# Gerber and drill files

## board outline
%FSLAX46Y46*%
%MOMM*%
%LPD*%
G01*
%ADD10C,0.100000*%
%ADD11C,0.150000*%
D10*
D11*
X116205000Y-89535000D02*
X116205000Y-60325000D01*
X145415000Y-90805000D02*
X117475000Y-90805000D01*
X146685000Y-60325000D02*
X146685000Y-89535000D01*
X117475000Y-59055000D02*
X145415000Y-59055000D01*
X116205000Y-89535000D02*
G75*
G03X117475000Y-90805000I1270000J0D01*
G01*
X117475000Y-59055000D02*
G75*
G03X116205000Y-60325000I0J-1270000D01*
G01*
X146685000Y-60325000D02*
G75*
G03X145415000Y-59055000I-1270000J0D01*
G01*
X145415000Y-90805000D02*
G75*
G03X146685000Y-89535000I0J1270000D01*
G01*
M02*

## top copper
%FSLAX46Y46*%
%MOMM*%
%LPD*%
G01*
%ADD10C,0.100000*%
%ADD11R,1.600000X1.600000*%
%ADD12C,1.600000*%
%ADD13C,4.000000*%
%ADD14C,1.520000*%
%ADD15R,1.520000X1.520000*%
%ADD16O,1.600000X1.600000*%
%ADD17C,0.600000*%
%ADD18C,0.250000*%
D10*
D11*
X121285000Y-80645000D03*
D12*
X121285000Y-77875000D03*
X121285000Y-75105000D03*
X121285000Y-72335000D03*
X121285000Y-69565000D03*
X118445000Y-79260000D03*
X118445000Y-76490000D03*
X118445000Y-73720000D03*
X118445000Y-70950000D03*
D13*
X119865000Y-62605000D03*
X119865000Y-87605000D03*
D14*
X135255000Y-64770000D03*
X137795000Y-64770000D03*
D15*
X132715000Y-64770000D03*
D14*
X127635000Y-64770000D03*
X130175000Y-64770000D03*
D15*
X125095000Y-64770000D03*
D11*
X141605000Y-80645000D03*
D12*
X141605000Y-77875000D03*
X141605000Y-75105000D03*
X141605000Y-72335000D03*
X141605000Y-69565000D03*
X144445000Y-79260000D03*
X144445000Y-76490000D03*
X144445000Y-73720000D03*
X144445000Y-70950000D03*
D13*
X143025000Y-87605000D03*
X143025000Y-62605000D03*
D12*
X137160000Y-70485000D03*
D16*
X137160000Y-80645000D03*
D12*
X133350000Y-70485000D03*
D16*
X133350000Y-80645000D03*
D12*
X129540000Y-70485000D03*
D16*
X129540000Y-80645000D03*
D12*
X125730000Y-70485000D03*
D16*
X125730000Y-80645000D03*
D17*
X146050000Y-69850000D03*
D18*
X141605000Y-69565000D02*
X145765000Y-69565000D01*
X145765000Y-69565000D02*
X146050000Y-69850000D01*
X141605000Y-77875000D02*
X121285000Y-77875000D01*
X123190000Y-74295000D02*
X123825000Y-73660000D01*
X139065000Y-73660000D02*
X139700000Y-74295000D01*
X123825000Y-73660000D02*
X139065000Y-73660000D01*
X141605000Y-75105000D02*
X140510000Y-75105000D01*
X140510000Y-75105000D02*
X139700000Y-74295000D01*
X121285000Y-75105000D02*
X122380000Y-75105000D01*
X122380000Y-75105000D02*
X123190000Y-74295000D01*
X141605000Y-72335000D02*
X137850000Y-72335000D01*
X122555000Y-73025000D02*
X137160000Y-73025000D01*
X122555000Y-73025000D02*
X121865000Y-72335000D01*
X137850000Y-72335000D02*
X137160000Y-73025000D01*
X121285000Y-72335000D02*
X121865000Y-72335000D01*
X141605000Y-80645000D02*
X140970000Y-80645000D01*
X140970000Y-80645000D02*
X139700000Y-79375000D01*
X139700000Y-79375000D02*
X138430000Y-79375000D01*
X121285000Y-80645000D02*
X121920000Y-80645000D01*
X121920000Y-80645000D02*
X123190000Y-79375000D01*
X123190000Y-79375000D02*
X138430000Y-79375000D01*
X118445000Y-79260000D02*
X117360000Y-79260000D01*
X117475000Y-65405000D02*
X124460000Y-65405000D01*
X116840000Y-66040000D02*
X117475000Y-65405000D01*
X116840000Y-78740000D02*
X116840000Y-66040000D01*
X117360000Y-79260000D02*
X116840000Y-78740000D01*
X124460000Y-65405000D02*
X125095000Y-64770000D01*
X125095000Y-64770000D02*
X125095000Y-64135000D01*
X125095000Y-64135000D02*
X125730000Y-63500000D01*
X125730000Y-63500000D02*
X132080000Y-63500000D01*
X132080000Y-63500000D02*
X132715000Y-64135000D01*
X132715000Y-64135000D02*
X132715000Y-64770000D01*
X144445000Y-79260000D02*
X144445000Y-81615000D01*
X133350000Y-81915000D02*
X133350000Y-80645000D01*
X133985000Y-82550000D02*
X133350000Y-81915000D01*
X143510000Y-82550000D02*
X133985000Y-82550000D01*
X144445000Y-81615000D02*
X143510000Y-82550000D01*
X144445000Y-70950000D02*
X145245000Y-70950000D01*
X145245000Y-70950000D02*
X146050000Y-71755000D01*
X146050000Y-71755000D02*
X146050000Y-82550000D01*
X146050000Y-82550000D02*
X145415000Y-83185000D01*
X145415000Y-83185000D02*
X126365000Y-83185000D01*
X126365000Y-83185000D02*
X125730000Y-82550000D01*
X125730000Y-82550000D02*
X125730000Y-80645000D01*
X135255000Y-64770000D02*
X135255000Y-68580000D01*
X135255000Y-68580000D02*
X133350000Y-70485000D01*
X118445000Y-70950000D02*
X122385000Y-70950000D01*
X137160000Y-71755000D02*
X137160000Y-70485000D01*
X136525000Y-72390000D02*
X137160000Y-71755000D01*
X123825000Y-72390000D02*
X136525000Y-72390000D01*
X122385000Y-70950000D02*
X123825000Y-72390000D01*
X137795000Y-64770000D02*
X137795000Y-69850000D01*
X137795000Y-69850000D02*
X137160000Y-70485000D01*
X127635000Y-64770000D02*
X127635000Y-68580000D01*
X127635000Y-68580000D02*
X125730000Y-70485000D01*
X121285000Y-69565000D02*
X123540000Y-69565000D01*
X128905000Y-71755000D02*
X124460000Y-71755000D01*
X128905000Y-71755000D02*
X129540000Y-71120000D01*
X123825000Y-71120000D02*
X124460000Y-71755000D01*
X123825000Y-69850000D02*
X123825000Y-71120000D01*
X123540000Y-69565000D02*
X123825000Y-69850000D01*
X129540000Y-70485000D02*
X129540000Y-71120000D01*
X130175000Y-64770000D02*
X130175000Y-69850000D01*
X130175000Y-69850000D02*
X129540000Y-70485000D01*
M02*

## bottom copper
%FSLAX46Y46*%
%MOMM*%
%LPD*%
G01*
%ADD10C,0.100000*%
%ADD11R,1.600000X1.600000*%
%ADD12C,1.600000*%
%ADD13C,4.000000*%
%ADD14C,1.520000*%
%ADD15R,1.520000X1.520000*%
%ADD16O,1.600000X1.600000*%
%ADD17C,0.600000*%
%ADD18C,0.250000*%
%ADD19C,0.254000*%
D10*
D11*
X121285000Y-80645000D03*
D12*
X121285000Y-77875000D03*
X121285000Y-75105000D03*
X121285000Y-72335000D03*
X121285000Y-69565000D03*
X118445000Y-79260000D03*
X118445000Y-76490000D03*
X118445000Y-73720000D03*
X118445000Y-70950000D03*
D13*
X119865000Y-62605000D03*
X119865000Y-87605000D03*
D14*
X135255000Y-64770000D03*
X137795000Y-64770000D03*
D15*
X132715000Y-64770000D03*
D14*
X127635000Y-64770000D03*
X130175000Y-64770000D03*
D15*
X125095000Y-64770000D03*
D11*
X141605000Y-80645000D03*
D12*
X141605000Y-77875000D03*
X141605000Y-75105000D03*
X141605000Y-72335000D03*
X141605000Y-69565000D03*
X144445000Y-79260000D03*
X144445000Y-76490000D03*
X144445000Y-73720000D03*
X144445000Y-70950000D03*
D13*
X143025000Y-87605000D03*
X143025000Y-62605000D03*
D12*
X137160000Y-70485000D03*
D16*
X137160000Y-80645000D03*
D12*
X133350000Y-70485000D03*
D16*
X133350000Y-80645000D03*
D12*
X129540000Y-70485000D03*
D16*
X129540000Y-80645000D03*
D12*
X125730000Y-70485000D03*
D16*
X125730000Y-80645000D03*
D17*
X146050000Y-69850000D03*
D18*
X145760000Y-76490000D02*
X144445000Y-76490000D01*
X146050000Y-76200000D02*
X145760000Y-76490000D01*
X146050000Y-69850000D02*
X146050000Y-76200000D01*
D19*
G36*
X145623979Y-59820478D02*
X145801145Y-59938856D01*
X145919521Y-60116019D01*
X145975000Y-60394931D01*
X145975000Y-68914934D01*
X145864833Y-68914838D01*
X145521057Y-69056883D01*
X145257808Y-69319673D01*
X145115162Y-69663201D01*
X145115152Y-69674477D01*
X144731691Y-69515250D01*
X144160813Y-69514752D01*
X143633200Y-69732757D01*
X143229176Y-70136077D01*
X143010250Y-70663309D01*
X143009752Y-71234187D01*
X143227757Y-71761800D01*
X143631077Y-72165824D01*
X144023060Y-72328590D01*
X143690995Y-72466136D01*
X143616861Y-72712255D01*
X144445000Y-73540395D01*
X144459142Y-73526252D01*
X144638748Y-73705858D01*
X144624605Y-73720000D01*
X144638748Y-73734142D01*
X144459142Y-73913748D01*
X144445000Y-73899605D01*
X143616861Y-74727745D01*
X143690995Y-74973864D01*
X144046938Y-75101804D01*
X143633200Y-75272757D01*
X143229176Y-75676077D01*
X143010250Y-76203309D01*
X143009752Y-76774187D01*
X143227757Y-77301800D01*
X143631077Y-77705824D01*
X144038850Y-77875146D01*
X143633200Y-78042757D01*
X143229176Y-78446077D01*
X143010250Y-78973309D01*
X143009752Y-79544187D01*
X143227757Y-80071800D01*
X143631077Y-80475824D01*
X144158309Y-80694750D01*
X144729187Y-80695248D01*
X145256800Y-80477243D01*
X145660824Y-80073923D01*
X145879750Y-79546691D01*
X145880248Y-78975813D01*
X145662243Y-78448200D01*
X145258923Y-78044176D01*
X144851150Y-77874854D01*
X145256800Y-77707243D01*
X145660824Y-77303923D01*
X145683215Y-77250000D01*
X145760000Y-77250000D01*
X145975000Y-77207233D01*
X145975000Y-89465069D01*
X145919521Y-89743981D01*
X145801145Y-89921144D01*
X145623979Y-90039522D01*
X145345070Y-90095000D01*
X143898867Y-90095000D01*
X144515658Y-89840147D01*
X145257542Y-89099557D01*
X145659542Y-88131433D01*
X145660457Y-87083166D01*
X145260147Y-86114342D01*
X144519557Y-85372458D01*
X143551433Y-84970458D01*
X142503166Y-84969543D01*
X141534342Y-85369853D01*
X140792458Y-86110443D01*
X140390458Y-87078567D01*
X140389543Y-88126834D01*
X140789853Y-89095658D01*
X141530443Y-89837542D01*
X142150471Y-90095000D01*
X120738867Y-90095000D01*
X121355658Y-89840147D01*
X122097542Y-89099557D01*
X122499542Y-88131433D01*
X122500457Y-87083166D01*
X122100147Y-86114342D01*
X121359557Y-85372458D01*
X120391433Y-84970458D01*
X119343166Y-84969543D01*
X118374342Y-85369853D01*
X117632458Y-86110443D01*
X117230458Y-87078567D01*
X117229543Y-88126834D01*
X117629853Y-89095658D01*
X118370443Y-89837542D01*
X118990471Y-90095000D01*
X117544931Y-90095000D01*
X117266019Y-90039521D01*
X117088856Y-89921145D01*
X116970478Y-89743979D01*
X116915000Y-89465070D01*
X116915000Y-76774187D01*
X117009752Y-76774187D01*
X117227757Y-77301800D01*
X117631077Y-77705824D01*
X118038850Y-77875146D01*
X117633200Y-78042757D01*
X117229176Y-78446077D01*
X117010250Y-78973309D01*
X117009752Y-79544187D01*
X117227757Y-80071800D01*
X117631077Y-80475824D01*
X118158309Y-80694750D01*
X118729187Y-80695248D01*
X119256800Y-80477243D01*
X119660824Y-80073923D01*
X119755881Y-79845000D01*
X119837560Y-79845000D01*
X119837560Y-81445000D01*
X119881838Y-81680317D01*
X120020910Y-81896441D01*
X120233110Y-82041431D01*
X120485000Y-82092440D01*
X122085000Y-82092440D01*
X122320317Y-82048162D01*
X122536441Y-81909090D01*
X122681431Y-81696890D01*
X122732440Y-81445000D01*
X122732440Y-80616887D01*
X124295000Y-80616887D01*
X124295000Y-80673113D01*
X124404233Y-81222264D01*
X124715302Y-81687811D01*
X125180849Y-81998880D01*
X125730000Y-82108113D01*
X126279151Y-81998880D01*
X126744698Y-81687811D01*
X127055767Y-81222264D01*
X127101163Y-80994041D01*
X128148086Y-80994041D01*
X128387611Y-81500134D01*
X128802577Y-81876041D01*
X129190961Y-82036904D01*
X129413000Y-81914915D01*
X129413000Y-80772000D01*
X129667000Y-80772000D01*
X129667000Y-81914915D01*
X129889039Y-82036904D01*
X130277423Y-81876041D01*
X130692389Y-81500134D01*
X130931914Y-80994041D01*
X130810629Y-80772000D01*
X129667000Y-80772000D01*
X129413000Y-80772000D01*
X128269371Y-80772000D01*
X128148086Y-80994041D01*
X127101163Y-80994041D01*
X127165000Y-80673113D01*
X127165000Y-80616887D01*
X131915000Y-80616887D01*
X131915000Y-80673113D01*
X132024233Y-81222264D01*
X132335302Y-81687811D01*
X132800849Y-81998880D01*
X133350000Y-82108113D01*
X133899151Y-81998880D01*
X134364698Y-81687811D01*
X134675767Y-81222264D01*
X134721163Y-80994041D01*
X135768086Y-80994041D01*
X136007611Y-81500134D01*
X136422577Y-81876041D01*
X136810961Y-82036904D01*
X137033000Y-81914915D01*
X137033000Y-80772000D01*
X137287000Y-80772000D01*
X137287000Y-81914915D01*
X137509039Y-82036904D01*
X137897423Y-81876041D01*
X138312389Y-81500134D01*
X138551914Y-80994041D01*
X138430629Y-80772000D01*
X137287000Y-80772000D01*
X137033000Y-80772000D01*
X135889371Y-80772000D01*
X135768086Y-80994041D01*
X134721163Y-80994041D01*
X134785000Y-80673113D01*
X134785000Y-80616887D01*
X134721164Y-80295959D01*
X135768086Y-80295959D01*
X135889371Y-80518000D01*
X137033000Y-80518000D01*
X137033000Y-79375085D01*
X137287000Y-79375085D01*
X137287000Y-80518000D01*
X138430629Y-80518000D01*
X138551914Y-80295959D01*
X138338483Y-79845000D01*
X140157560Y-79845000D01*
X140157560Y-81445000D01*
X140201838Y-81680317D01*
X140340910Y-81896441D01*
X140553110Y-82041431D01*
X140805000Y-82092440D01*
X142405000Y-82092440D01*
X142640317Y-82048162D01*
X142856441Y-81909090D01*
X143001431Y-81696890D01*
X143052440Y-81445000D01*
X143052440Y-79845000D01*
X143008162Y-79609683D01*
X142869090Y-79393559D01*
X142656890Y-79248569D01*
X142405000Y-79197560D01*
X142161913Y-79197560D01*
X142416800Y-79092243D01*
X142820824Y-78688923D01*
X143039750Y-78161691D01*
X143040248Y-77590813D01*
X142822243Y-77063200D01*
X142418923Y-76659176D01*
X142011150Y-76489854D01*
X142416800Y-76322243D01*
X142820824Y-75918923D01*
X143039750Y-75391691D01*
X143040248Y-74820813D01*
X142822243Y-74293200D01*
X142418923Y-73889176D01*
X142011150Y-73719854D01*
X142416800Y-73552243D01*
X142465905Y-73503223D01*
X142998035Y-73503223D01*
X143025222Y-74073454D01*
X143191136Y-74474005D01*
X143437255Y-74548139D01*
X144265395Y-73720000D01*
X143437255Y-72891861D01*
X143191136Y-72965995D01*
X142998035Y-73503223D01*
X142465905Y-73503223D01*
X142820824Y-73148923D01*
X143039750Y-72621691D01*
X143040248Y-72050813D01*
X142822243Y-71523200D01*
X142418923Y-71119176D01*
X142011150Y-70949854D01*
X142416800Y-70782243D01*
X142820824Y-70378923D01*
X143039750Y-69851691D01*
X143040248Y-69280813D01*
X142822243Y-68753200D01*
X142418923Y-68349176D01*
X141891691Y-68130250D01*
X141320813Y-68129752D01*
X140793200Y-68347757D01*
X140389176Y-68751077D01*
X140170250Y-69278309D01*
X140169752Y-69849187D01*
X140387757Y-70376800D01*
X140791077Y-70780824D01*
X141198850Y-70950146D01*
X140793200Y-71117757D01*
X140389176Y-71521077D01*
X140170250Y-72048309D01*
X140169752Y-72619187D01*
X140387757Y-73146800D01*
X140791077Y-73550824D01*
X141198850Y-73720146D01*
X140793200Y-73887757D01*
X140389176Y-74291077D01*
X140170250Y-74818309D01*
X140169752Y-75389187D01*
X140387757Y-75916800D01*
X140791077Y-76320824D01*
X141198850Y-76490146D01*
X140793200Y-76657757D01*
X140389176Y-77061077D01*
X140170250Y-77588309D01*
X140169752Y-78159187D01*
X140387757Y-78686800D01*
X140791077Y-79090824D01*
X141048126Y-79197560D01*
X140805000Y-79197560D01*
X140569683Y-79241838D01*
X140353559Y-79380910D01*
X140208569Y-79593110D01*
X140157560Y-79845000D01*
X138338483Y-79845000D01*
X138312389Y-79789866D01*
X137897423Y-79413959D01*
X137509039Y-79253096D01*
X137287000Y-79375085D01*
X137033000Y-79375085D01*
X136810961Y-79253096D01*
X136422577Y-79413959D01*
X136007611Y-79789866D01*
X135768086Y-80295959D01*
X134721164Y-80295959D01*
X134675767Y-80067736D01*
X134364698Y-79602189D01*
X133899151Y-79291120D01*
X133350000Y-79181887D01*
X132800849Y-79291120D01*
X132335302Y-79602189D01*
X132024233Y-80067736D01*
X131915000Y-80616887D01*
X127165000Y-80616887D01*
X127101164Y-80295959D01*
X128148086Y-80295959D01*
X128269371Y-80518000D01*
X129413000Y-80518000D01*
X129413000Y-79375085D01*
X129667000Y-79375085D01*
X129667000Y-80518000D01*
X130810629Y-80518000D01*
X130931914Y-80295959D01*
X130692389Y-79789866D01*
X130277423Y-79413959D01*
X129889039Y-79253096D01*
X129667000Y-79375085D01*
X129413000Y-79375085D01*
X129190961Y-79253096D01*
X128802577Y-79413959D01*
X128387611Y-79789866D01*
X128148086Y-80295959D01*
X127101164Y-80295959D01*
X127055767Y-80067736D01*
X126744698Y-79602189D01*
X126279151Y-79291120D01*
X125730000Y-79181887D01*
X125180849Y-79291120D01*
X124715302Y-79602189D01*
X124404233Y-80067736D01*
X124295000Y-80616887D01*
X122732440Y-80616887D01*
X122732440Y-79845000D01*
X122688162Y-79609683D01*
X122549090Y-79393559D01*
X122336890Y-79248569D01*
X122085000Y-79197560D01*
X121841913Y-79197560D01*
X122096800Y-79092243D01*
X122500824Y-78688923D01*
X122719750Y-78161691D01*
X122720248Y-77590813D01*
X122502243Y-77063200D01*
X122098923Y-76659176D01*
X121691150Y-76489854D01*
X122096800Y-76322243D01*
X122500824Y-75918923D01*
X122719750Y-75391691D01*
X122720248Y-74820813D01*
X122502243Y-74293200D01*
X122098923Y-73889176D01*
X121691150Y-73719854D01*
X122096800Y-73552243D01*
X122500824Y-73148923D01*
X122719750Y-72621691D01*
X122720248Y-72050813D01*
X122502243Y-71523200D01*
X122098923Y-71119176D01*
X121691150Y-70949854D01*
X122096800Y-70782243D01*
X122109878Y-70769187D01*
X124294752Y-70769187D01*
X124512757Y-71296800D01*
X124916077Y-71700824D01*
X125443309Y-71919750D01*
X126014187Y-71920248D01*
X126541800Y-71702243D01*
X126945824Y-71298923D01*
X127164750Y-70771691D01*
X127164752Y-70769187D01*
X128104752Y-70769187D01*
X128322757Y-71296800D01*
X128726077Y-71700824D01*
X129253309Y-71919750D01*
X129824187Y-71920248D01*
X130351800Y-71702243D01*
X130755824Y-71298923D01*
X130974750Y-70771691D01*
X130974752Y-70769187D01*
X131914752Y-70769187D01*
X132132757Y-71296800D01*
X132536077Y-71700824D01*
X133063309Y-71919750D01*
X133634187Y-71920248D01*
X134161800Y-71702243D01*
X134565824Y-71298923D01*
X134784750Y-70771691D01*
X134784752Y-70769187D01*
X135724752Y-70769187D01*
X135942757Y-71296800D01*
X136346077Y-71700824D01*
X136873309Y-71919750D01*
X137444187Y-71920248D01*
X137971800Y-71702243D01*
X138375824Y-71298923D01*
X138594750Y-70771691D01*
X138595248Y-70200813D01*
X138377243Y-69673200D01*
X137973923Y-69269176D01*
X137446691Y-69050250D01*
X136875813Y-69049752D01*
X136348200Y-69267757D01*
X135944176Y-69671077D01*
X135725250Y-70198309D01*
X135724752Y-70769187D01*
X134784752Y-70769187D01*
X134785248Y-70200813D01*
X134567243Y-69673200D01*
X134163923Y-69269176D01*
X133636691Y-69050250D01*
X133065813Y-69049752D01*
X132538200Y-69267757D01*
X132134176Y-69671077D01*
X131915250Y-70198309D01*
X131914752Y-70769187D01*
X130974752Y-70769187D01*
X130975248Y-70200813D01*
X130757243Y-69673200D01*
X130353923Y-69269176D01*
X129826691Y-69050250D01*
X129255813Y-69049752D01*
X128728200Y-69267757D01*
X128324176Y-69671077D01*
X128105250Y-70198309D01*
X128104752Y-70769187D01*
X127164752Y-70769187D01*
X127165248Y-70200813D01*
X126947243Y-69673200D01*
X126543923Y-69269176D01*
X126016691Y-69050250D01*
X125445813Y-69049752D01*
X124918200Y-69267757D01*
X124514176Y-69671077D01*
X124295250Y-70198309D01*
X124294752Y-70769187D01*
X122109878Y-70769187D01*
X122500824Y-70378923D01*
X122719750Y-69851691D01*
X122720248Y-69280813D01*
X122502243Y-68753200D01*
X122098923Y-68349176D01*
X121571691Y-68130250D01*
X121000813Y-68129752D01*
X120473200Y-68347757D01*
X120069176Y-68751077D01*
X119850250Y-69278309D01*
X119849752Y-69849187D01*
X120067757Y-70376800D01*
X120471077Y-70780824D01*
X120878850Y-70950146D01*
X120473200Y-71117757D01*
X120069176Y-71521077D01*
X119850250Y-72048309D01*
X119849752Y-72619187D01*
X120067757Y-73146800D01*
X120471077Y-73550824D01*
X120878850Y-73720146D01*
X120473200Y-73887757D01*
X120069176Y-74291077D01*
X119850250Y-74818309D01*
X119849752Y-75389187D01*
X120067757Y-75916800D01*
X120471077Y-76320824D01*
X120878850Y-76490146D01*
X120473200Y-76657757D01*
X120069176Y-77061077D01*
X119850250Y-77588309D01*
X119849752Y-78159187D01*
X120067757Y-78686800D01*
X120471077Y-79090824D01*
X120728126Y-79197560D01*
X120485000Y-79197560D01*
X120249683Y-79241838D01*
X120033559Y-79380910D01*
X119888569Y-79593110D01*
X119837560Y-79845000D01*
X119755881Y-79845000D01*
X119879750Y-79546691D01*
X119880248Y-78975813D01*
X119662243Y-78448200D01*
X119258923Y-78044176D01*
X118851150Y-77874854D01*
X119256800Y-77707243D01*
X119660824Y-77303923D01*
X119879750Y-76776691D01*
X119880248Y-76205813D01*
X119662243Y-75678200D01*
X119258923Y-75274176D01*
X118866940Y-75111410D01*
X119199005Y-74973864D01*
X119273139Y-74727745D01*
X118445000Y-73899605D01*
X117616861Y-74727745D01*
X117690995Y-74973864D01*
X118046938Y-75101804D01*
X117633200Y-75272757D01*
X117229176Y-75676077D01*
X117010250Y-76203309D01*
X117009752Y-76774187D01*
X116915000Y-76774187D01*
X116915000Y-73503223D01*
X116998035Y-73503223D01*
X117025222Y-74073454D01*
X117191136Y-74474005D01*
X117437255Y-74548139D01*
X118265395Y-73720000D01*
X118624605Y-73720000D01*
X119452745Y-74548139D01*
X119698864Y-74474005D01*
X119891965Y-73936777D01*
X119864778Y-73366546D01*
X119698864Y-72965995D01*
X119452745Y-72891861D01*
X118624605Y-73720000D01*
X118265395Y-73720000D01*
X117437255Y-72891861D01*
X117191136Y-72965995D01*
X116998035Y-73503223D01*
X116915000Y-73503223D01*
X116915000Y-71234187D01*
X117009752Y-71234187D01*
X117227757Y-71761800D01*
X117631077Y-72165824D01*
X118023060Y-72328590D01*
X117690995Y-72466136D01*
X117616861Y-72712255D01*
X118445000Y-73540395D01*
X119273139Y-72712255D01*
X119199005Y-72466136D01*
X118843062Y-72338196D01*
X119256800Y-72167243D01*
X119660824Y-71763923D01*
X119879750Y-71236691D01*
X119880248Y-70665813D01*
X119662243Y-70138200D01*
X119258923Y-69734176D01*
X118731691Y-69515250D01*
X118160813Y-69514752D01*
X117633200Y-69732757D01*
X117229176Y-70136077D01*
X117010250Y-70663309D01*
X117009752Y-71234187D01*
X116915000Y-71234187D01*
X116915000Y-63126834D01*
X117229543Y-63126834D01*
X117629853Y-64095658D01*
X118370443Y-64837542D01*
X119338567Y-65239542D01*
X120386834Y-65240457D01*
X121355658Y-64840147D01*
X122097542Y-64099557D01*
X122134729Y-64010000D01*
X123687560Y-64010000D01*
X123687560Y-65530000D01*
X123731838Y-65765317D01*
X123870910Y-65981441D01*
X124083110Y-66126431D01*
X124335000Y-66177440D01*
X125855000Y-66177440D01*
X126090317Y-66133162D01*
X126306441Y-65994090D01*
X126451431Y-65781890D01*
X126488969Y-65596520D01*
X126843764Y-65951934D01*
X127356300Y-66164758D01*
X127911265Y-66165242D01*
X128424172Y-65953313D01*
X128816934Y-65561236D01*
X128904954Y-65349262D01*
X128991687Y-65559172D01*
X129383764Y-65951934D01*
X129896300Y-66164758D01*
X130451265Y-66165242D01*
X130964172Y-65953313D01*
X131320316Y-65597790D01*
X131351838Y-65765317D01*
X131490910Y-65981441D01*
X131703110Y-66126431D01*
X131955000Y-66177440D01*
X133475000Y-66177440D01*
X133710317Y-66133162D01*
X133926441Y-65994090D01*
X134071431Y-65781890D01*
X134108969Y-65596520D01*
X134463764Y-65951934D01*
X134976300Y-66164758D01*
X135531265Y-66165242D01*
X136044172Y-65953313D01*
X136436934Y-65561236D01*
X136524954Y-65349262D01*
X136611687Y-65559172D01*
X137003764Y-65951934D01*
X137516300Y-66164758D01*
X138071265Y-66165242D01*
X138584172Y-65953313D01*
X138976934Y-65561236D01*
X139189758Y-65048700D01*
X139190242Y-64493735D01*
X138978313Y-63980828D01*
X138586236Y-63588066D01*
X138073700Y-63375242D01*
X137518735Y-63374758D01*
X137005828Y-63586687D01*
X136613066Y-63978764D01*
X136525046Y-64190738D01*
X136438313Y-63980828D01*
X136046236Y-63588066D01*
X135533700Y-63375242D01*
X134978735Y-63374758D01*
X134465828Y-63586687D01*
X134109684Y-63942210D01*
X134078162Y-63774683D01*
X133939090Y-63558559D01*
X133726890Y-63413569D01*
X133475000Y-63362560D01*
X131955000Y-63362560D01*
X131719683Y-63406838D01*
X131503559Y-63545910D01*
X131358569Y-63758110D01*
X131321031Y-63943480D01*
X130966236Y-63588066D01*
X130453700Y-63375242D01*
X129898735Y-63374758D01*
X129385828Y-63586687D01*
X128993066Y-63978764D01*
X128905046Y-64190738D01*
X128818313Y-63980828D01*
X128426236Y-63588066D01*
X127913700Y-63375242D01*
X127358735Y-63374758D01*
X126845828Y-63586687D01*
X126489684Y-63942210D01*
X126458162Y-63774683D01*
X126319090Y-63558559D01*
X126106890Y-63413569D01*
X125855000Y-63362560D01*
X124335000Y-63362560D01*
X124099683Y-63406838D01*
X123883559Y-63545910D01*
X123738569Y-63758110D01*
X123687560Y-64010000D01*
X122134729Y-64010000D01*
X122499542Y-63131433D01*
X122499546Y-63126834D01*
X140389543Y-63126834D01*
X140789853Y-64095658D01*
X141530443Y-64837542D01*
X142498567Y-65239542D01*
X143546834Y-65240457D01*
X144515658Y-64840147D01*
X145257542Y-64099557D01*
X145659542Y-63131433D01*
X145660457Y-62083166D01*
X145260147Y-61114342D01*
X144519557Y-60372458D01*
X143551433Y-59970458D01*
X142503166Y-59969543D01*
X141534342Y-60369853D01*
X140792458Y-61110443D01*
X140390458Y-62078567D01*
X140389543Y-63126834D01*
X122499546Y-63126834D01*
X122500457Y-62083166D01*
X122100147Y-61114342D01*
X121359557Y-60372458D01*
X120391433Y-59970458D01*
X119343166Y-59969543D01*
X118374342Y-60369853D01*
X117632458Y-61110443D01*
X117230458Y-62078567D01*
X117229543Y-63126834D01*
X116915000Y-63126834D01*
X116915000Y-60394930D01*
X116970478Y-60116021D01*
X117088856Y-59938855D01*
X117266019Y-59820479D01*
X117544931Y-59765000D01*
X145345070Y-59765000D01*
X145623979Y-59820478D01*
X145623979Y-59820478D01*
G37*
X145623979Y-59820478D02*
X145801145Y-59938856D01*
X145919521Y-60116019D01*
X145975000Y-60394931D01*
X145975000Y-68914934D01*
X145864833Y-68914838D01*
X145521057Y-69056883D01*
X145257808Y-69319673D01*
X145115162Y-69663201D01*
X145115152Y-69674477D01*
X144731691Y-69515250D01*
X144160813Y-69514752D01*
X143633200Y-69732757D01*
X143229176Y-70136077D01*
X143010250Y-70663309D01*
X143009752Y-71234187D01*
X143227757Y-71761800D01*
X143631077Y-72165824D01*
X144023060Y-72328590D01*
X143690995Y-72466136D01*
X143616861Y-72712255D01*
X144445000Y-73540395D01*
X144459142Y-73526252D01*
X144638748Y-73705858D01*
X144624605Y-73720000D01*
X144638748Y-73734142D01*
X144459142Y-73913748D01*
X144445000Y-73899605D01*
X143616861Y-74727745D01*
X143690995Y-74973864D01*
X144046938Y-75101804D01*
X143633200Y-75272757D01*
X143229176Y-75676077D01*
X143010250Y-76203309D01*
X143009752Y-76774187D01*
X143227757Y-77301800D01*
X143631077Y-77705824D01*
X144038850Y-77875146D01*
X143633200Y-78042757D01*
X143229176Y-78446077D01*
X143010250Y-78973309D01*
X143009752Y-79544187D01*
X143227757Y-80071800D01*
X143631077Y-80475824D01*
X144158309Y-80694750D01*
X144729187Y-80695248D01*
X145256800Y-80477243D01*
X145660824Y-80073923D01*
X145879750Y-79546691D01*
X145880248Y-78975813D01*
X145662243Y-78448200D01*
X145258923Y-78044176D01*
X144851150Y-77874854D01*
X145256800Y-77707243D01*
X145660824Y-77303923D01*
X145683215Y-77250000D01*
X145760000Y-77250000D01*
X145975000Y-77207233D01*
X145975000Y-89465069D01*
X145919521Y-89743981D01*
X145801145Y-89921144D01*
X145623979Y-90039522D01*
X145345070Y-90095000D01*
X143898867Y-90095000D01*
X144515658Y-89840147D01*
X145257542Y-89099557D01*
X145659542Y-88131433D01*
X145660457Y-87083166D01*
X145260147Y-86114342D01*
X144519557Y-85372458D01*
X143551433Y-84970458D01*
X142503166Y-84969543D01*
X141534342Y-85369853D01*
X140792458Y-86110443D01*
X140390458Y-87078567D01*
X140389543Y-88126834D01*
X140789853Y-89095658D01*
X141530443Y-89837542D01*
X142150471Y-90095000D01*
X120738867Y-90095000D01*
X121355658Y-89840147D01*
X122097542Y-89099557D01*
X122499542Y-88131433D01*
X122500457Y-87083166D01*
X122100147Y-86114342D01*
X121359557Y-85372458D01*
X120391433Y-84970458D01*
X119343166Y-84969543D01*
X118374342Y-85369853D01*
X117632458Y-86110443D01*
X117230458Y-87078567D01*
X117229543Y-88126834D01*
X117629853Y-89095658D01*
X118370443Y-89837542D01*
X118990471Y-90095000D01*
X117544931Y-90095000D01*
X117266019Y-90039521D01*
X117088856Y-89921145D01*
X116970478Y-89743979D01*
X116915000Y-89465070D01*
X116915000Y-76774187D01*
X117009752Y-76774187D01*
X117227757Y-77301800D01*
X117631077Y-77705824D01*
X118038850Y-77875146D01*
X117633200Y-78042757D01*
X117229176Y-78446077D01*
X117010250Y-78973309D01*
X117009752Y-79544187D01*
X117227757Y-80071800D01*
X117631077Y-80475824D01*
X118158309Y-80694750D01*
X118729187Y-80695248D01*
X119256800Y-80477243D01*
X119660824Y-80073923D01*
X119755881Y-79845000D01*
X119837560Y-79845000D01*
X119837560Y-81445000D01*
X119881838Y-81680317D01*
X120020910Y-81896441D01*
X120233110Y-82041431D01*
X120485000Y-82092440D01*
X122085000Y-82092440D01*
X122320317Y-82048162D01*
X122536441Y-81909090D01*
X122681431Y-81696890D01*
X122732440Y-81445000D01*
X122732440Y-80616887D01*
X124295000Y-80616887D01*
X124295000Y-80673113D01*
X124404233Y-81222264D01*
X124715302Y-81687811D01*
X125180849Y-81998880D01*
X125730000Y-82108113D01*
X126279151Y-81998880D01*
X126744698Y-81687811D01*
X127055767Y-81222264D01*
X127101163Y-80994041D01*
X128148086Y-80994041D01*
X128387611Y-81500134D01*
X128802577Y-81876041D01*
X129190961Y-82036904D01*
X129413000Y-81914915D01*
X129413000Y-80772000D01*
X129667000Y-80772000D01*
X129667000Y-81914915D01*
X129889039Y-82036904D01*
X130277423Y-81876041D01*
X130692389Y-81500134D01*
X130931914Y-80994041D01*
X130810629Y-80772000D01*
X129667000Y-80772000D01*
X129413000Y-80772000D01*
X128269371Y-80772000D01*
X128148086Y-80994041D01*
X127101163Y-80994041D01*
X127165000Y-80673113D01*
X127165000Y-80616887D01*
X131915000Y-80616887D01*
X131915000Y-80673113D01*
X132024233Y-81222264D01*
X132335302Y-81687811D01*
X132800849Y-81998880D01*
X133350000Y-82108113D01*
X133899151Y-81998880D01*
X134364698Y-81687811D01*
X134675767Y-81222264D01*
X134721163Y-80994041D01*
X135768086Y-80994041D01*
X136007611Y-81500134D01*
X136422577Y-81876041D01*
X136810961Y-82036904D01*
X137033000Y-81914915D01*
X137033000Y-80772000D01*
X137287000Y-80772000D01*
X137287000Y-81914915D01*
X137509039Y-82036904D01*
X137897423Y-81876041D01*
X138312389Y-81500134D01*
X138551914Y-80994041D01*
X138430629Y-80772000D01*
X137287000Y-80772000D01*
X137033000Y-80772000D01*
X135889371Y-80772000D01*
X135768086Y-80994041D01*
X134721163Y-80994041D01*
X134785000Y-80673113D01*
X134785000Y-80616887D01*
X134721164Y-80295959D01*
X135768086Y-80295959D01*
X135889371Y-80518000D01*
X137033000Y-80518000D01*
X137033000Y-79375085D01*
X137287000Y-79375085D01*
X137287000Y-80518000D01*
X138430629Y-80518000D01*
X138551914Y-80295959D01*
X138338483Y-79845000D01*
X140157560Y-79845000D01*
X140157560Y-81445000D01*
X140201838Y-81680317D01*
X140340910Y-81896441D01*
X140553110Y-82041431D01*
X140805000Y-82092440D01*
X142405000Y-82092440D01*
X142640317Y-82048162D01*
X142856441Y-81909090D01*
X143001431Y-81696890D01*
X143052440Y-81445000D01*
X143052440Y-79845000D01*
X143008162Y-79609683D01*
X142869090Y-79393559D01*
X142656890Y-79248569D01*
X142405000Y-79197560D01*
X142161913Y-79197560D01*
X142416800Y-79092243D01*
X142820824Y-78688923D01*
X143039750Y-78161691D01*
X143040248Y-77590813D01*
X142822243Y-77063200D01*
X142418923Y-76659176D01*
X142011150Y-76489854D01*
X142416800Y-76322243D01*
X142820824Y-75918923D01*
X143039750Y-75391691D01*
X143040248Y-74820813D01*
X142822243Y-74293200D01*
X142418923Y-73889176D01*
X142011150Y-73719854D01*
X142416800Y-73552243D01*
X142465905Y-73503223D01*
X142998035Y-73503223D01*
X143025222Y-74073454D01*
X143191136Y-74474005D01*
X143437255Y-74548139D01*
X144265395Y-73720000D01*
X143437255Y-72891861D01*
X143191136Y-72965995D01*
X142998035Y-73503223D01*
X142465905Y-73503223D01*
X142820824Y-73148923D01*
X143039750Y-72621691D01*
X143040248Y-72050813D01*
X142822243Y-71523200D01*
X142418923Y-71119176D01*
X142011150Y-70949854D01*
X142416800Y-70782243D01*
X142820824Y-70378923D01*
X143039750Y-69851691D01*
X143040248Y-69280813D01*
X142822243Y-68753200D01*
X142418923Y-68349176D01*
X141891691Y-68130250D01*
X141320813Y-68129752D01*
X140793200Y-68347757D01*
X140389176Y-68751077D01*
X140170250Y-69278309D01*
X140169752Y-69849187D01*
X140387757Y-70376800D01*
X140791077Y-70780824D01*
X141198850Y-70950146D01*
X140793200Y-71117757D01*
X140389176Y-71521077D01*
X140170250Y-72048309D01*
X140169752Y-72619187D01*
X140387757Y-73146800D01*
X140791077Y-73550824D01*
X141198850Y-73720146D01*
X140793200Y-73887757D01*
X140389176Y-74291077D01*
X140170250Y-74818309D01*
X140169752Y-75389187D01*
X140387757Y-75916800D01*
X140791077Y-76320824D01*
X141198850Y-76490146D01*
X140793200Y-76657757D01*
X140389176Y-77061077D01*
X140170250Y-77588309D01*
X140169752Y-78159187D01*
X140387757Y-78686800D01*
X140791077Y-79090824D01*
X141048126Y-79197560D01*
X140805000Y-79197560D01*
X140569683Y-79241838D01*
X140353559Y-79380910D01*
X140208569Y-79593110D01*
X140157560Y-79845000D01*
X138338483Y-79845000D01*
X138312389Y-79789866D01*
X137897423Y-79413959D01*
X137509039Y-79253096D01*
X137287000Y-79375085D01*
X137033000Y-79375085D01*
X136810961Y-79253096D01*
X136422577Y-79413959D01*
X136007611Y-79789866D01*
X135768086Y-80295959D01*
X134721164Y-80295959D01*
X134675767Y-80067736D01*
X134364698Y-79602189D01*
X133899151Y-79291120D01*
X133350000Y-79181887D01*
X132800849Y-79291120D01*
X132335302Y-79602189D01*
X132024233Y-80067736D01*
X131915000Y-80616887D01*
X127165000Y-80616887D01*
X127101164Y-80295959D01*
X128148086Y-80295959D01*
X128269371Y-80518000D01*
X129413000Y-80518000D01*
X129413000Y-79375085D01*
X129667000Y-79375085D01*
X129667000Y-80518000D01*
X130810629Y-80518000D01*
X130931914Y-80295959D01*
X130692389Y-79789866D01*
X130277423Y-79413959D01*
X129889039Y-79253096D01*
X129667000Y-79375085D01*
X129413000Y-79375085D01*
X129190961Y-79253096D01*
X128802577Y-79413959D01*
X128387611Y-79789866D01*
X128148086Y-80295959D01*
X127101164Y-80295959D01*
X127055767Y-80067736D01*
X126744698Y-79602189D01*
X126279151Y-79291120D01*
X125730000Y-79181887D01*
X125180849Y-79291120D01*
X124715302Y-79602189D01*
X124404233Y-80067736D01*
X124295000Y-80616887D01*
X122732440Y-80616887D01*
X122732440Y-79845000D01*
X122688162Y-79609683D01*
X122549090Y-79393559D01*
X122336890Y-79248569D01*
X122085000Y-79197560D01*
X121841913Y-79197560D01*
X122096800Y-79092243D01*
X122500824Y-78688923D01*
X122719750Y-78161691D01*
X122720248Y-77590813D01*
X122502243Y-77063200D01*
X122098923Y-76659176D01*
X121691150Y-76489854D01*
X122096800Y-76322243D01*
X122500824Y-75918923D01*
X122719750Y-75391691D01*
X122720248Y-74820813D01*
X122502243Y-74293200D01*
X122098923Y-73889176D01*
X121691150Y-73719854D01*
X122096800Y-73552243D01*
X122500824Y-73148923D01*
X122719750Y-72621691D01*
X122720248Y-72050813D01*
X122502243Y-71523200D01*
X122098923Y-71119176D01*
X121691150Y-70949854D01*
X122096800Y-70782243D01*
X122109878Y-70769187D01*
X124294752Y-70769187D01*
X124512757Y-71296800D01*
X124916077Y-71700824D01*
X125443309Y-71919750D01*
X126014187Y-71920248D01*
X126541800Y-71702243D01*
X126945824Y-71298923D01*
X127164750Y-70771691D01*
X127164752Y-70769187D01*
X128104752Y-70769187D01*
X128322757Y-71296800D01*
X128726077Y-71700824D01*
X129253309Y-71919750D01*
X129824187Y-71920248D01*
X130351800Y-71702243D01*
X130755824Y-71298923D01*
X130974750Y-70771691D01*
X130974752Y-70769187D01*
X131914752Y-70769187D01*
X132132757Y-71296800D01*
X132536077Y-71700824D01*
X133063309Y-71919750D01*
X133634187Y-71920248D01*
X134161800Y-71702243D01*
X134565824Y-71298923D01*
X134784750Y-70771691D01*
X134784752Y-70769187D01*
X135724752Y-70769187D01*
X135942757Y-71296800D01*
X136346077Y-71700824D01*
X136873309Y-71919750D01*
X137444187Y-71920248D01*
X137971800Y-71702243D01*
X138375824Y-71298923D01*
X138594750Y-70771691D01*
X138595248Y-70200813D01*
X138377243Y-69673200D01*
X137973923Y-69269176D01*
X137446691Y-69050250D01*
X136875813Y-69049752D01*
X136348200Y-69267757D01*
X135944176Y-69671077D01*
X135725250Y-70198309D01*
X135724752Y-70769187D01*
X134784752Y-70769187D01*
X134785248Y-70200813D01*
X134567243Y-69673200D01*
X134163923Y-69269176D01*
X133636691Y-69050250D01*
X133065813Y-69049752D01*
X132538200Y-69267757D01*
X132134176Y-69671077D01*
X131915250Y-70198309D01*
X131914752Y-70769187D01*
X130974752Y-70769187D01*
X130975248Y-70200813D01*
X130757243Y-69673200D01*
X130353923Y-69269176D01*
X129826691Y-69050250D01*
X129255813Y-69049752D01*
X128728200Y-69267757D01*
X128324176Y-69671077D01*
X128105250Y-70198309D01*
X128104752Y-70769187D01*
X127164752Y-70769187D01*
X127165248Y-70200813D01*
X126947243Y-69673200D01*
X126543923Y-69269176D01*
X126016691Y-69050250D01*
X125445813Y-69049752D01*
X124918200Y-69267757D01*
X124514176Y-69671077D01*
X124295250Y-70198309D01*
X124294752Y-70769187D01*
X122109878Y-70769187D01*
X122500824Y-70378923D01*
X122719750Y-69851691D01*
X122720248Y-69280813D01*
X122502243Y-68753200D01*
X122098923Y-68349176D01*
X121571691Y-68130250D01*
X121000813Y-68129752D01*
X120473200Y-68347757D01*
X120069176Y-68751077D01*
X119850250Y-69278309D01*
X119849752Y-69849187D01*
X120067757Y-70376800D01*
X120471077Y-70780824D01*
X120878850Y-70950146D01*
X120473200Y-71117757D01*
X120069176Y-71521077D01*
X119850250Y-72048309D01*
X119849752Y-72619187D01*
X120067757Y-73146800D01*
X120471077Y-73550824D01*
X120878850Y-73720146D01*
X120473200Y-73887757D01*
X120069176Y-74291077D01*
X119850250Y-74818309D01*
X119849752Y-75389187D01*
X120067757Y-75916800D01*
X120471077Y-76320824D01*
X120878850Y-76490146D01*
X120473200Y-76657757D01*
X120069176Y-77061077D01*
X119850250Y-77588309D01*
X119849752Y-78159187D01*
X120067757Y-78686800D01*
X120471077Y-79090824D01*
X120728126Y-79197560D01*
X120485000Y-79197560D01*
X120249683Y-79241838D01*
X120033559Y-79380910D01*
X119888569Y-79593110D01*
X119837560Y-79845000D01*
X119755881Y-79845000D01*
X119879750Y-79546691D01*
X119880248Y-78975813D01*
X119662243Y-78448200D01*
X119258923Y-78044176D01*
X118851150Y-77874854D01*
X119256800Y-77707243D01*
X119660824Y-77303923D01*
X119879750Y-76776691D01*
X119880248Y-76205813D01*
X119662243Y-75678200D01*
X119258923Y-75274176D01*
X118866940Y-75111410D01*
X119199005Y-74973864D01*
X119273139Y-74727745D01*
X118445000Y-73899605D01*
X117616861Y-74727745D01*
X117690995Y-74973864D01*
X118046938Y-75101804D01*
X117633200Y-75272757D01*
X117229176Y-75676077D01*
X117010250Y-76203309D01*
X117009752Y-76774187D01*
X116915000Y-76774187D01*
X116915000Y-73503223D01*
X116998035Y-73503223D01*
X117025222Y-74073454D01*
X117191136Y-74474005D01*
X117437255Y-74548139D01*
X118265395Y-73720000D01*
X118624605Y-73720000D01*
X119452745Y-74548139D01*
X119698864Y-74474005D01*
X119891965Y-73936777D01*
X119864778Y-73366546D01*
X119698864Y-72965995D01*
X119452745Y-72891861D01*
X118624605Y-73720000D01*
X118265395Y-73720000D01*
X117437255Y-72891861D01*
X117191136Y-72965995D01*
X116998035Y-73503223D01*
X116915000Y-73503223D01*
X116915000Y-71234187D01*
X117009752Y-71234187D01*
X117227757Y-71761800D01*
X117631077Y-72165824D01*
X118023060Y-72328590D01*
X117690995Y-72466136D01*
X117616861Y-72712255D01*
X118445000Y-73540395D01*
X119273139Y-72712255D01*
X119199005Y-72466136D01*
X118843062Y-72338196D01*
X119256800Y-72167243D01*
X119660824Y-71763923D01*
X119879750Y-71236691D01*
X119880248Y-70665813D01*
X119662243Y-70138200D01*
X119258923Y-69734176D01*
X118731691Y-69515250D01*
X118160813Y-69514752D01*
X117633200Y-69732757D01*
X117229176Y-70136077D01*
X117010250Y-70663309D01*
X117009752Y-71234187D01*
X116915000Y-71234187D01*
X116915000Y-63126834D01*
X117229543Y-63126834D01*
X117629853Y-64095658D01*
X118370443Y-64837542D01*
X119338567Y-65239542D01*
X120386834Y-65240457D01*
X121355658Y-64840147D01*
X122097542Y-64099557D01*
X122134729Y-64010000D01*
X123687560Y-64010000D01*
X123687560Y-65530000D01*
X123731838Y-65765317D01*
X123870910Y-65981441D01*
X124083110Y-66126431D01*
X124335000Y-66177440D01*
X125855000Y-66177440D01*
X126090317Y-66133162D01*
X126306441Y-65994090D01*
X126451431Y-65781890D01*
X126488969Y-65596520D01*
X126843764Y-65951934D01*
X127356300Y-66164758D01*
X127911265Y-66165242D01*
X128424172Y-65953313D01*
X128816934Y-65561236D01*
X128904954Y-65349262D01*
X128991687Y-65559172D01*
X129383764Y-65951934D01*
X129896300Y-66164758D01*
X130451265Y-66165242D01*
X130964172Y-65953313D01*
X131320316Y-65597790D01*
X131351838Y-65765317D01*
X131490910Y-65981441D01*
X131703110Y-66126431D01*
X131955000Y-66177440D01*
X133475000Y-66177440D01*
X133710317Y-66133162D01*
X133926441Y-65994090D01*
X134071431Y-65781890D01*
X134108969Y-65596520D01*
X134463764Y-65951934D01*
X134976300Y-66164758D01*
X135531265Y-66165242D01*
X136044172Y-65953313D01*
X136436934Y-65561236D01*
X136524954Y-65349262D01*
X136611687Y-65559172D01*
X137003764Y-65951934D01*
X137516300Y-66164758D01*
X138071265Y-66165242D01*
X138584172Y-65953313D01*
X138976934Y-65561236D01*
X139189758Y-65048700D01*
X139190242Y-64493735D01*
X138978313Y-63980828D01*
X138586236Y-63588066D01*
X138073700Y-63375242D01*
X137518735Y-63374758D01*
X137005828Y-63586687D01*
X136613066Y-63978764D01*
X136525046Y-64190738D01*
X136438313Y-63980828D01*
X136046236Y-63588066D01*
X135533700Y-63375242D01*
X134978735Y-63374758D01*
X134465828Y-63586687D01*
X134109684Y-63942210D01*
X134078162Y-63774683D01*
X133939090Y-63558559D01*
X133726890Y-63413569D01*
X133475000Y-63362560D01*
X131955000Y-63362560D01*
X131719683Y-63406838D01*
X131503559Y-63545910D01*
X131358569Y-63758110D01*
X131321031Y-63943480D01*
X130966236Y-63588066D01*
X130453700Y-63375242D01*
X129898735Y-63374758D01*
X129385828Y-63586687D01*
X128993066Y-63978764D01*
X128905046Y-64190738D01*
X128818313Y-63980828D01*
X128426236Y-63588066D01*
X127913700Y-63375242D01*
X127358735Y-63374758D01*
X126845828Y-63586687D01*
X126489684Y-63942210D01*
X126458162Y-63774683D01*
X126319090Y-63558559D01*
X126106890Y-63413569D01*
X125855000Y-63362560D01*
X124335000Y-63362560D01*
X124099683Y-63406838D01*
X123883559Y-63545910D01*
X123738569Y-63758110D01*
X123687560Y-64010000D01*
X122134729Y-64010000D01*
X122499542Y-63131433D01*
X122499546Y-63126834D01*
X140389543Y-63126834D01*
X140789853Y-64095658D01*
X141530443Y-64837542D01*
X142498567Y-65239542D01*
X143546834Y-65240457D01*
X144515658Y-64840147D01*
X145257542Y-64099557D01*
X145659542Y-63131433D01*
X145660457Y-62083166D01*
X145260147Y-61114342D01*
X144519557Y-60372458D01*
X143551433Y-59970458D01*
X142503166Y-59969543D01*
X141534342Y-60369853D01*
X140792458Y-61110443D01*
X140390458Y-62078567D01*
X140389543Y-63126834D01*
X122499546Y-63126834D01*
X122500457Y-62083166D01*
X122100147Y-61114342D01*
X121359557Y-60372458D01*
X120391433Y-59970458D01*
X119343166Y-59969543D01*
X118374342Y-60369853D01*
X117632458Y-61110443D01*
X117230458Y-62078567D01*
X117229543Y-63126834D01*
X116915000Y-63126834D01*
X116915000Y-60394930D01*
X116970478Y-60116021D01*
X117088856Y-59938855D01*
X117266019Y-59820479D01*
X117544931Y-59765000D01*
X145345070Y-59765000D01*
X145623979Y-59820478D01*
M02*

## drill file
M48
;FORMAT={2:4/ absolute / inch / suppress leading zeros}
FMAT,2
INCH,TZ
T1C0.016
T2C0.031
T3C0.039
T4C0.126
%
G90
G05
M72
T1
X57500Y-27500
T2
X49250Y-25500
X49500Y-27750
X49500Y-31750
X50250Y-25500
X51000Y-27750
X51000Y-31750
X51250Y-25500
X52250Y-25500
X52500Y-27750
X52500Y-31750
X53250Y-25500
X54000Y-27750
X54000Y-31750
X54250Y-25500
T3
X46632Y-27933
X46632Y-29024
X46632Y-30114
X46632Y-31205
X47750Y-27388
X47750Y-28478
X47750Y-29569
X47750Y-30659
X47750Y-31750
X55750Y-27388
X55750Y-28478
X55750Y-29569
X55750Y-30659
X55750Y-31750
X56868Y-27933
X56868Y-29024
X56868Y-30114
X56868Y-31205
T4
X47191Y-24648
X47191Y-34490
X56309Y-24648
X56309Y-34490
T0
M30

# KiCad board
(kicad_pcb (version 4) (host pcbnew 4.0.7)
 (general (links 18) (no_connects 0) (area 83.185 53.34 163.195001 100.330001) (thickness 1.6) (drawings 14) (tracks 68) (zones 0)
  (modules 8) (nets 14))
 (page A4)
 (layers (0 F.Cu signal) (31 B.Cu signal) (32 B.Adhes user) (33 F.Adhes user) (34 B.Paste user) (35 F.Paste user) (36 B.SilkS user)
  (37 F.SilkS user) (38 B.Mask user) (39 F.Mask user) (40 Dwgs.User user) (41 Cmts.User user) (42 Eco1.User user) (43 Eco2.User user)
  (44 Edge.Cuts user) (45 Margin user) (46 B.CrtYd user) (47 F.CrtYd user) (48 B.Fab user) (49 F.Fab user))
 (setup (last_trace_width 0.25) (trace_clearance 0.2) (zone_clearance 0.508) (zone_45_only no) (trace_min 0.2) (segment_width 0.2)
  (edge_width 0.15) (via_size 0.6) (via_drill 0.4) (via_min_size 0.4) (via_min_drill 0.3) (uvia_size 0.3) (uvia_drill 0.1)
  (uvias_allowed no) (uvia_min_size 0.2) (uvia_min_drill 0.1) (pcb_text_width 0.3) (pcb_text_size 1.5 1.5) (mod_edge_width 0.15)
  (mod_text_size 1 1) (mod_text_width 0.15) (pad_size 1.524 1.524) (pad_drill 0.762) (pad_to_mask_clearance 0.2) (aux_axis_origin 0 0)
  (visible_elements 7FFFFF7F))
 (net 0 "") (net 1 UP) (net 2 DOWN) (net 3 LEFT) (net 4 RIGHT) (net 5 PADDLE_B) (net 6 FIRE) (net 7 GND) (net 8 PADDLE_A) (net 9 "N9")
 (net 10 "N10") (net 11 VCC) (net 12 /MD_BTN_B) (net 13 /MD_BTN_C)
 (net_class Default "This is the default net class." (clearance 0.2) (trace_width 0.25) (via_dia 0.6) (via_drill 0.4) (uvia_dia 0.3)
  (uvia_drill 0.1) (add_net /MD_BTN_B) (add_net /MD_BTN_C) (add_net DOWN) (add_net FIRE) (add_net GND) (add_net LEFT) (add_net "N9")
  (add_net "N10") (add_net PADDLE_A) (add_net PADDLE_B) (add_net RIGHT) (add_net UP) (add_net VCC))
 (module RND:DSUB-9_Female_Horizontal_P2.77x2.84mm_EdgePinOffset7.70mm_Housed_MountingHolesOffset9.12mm (layer F.Cu) (at 121.285 80.645 270)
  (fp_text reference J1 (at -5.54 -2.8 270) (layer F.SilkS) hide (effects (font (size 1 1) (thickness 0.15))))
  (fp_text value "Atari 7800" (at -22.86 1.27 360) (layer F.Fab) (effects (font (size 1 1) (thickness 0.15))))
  (pad 1 thru_hole rect (at 0 0 270) (size 1.6 1.6) (drill 1) (layers *.Cu *.Mask) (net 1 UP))
  (pad 2 thru_hole circle (at -2.77 0 270) (size 1.6 1.6) (drill 1) (layers *.Cu *.Mask) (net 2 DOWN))
  (pad 3 thru_hole circle (at -5.54 0 270) (size 1.6 1.6) (drill 1) (layers *.Cu *.Mask) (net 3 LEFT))
  (pad 4 thru_hole circle (at -8.31 0 270) (size 1.6 1.6) (drill 1) (layers *.Cu *.Mask) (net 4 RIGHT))
  (pad 5 thru_hole circle (at -11.08 0 270) (size 1.6 1.6) (drill 1) (layers *.Cu *.Mask) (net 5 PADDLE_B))
  (pad 6 thru_hole circle (at -1.385 2.84 270) (size 1.6 1.6) (drill 1) (layers *.Cu *.Mask) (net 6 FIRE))
  (pad 7 thru_hole circle (at -4.155 2.84 270) (size 1.6 1.6) (drill 1) (layers *.Cu *.Mask))
  (pad 8 thru_hole circle (at -6.925 2.84 270) (size 1.6 1.6) (drill 1) (layers *.Cu *.Mask) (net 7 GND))
  (pad 9 thru_hole circle (at -9.695 2.84 270) (size 1.6 1.6) (drill 1) (layers *.Cu *.Mask) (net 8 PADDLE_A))
  (pad 0 thru_hole circle (at -18.04 1.42 270) (size 4 4) (drill 3.2) (layers *.Cu *.Mask))
  (pad 0 thru_hole circle (at 6.96 1.42 270) (size 4 4) (drill 3.2) (layers *.Cu *.Mask)))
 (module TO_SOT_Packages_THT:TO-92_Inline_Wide (layer F.Cu) (at 132.715 64.77)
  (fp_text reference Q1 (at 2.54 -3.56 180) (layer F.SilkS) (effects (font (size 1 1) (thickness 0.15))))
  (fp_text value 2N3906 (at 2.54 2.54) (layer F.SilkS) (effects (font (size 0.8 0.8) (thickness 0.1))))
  (pad 2 thru_hole circle (at 2.54 0 90) (size 1.52 1.52) (drill 0.8) (layers *.Cu *.Mask) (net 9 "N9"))
  (pad 3 thru_hole circle (at 5.08 0 90) (size 1.52 1.52) (drill 0.8) (layers *.Cu *.Mask) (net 8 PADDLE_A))
  (pad 1 thru_hole rect (at 0 0 90) (size 1.52 1.52) (drill 0.8) (layers *.Cu *.Mask) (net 6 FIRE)))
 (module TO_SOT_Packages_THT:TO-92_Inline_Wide (layer F.Cu) (at 125.095 64.77)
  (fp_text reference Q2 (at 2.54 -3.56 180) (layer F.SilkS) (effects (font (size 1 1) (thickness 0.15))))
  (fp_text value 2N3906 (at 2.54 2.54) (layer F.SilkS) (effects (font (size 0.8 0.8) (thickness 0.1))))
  (pad 2 thru_hole circle (at 2.54 0 90) (size 1.52 1.52) (drill 0.8) (layers *.Cu *.Mask) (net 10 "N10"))
  (pad 3 thru_hole circle (at 5.08 0 90) (size 1.52 1.52) (drill 0.8) (layers *.Cu *.Mask) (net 5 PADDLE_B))
  (pad 1 thru_hole rect (at 0 0 90) (size 1.52 1.52) (drill 0.8) (layers *.Cu *.Mask) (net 6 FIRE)))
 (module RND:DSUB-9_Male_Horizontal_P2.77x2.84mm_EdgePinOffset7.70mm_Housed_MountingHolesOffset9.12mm (layer F.Cu) (at 141.605 80.645 90)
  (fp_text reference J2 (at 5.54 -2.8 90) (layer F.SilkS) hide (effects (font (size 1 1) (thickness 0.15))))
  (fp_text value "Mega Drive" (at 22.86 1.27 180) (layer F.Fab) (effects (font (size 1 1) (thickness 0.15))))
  (pad 1 thru_hole rect (at 0 0 90) (size 1.6 1.6) (drill 1) (layers *.Cu *.Mask) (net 1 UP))
  (pad 2 thru_hole circle (at 2.77 0 90) (size 1.6 1.6) (drill 1) (layers *.Cu *.Mask) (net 2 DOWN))
  (pad 3 thru_hole circle (at 5.54 0 90) (size 1.6 1.6) (drill 1) (layers *.Cu *.Mask) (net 3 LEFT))
  (pad 4 thru_hole circle (at 8.31 0 90) (size 1.6 1.6) (drill 1) (layers *.Cu *.Mask) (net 4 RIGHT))
  (pad 5 thru_hole circle (at 11.08 0 90) (size 1.6 1.6) (drill 1) (layers *.Cu *.Mask) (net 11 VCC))
  (pad 6 thru_hole circle (at 1.385 2.84 90) (size 1.6 1.6) (drill 1) (layers *.Cu *.Mask) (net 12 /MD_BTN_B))
  (pad 7 thru_hole circle (at 4.155 2.84 90) (size 1.6 1.6) (drill 1) (layers *.Cu *.Mask) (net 11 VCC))
  (pad 8 thru_hole circle (at 6.925 2.84 90) (size 1.6 1.6) (drill 1) (layers *.Cu *.Mask) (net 7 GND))
  (pad 9 thru_hole circle (at 9.695 2.84 90) (size 1.6 1.6) (drill 1) (layers *.Cu *.Mask) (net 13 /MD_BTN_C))
  (pad 0 thru_hole circle (at -6.96 1.42 90) (size 4 4) (drill 3.2) (layers *.Cu *.Mask))
  (pad 0 thru_hole circle (at 18.04 1.42 90) (size 4 4) (drill 3.2) (layers *.Cu *.Mask)))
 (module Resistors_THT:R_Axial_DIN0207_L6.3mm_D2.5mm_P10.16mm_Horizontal (layer F.Cu) (at 137.16 70.485 270)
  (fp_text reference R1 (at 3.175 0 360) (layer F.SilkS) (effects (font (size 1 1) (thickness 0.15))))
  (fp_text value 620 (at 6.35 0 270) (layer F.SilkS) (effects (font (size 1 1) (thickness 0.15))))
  (pad 1 thru_hole circle (at 0 0 270) (size 1.6 1.6) (drill 0.8) (layers *.Cu *.Mask) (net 8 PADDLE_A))
  (pad 2 thru_hole oval (at 10.16 0 270) (size 1.6 1.6) (drill 0.8) (layers *.Cu *.Mask) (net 7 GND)))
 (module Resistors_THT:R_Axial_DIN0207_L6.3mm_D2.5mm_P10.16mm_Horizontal (layer F.Cu) (at 133.35 70.485 270)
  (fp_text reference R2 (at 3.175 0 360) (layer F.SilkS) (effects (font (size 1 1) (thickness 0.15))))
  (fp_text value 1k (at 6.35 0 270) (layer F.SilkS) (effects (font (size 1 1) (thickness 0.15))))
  (pad 1 thru_hole circle (at 0 0 270) (size 1.6 1.6) (drill 0.8) (layers *.Cu *.Mask) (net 9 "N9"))
  (pad 2 thru_hole oval (at 10.16 0 270) (size 1.6 1.6) (drill 0.8) (layers *.Cu *.Mask) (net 12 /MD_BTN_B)))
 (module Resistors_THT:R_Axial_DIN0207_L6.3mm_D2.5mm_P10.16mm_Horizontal (layer F.Cu) (at 129.54 70.485 270)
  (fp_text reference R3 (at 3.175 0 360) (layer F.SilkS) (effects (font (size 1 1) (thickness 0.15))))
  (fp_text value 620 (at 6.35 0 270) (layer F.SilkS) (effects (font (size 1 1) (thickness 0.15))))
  (pad 1 thru_hole circle (at 0 0 270) (size 1.6 1.6) (drill 0.8) (layers *.Cu *.Mask) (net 5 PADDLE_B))
  (pad 2 thru_hole oval (at 10.16 0 270) (size 1.6 1.6) (drill 0.8) (layers *.Cu *.Mask) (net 7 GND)))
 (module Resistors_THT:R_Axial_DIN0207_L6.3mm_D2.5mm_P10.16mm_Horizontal (layer F.Cu) (at 125.73 70.485 270)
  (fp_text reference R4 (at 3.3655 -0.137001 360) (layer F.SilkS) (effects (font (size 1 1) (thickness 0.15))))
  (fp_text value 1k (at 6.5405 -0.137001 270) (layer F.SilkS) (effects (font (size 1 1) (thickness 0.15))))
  (pad 1 thru_hole circle (at 0 0 270) (size 1.6 1.6) (drill 0.8) (layers *.Cu *.Mask) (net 10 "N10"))
  (pad 2 thru_hole oval (at 10.16 0 270) (size 1.6 1.6) (drill 0.8) (layers *.Cu *.Mask) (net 13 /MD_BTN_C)))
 (gr_line (start 116.205 89.535) (end 116.205 60.325) (angle 90) (layer Edge.Cuts) (width 0.15))
 (gr_line (start 145.415 90.805) (end 117.475 90.805) (angle 90) (layer Edge.Cuts) (width 0.15))
 (gr_line (start 146.685 60.325) (end 146.685 89.535) (angle 90) (layer Edge.Cuts) (width 0.15))
 (gr_line (start 117.475 59.055) (end 145.415 59.055) (angle 90) (layer Edge.Cuts) (width 0.15))
 (gr_arc (start 117.475 89.535) (end 117.475 90.805) (angle 90) (layer Edge.Cuts) (width 0.15))
 (gr_arc (start 117.475 60.325) (end 116.205 60.325) (angle 90) (layer Edge.Cuts) (width 0.15))
 (gr_arc (start 145.415 60.325) (end 145.415 59.055) (angle 90) (layer Edge.Cuts) (width 0.15))
 (gr_arc (start 145.415 89.535) (end 146.685 89.535) (angle 90) (layer Edge.Cuts) (width 0.15))
 (segment (start 141.605 69.565) (end 145.765 69.565) (width 0.25) (layer F.Cu) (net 11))
 (segment (start 145.76 76.49) (end 144.445 76.49) (width 0.25) (layer B.Cu) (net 11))
 (segment (start 146.05 76.2) (end 145.76 76.49) (width 0.25) (layer B.Cu) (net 11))
 (segment (start 146.05 69.85) (end 146.05 76.2) (width 0.25) (layer B.Cu) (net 11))
 (via (at 146.05 69.85) (size 0.6) (drill 0.4) (layers F.Cu B.Cu) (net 11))
 (segment (start 145.765 69.565) (end 146.05 69.85) (width 0.25) (layer F.Cu) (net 11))
 (segment (start 141.605 77.875) (end 121.285 77.875) (width 0.25) (layer F.Cu) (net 2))
 (segment (start 123.19 74.295) (end 123.825 73.66) (width 0.25) (layer F.Cu) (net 3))
 (segment (start 139.065 73.66) (end 139.7 74.295) (width 0.25) (layer F.Cu) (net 3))
 (segment (start 123.825 73.66) (end 139.065 73.66) (width 0.25) (layer F.Cu) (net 3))
 (segment (start 141.605 75.105) (end 140.51 75.105) (width 0.25) (layer F.Cu) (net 3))
 (segment (start 140.51 75.105) (end 139.7 74.295) (width 0.25) (layer F.Cu) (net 3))
 (segment (start 121.285 75.105) (end 122.38 75.105) (width 0.25) (layer F.Cu) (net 3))
 (segment (start 122.38 75.105) (end 123.19 74.295) (width 0.25) (layer F.Cu) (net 3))
 (segment (start 141.605 72.335) (end 137.85 72.335) (width 0.25) (layer F.Cu) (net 4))
 (segment (start 122.555 73.025) (end 137.16 73.025) (width 0.25) (layer F.Cu) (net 4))
 (segment (start 122.555 73.025) (end 121.865 72.335) (width 0.25) (layer F.Cu) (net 4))
 (segment (start 137.85 72.335) (end 137.16 73.025) (width 0.25) (layer F.Cu) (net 4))
 (segment (start 121.285 72.335) (end 121.865 72.335) (width 0.25) (layer F.Cu) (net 4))
 (segment (start 141.605 80.645) (end 140.97 80.645) (width 0.25) (layer F.Cu) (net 1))
 (segment (start 140.97 80.645) (end 139.7 79.375) (width 0.25) (layer F.Cu) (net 1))
 (segment (start 139.7 79.375) (end 138.43 79.375) (width 0.25) (layer F.Cu) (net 1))
 (segment (start 121.285 80.645) (end 121.92 80.645) (width 0.25) (layer F.Cu) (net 1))
 (segment (start 121.92 80.645) (end 123.19 79.375) (width 0.25) (layer F.Cu) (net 1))
 (segment (start 123.19 79.375) (end 138.43 79.375) (width 0.25) (layer F.Cu) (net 1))
 (segment (start 118.445 79.26) (end 117.36 79.26) (width 0.25) (layer F.Cu) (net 6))
 (segment (start 117.475 65.405) (end 124.46 65.405) (width 0.25) (layer F.Cu) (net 6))
 (segment (start 116.84 66.04) (end 117.475 65.405) (width 0.25) (layer F.Cu) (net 6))
 (segment (start 116.84 78.74) (end 116.84 66.04) (width 0.25) (layer F.Cu) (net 6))
 (segment (start 117.36 79.26) (end 116.84 78.74) (width 0.25) (layer F.Cu) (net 6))
 (segment (start 124.46 65.405) (end 125.095 64.77) (width 0.25) (layer F.Cu) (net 6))
 (segment (start 125.095 64.77) (end 125.095 64.135) (width 0.25) (layer F.Cu) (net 6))
 (segment (start 125.095 64.135) (end 125.73 63.5) (width 0.25) (layer F.Cu) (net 6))
 (segment (start 125.73 63.5) (end 132.08 63.5) (width 0.25) (layer F.Cu) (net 6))
 (segment (start 132.08 63.5) (end 132.715 64.135) (width 0.25) (layer F.Cu) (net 6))
 (segment (start 132.715 64.135) (end 132.715 64.77) (width 0.25) (layer F.Cu) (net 6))
 (segment (start 144.445 79.26) (end 144.445 81.615) (width 0.25) (layer F.Cu) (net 12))
 (segment (start 133.35 81.915) (end 133.35 80.645) (width 0.25) (layer F.Cu) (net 12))
 (segment (start 133.985 82.55) (end 133.35 81.915) (width 0.25) (layer F.Cu) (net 12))
 (segment (start 143.51 82.55) (end 133.985 82.55) (width 0.25) (layer F.Cu) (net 12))
 (segment (start 144.445 81.615) (end 143.51 82.55) (width 0.25) (layer F.Cu) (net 12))
 (segment (start 144.445 70.95) (end 145.245 70.95) (width 0.25) (layer F.Cu) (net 13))
 (segment (start 145.245 70.95) (end 146.05 71.755) (width 0.25) (layer F.Cu) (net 13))
 (segment (start 146.05 71.755) (end 146.05 82.55) (width 0.25) (layer F.Cu) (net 13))
 (segment (start 146.05 82.55) (end 145.415 83.185) (width 0.25) (layer F.Cu) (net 13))
 (segment (start 145.415 83.185) (end 126.365 83.185) (width 0.25) (layer F.Cu) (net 13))
 (segment (start 126.365 83.185) (end 125.73 82.55) (width 0.25) (layer F.Cu) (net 13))
 (segment (start 125.73 82.55) (end 125.73 80.645) (width 0.25) (layer F.Cu) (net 13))
 (segment (start 135.255 64.77) (end 135.255 68.58) (width 0.25) (layer F.Cu) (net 9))
 (segment (start 135.255 68.58) (end 133.35 70.485) (width 0.25) (layer F.Cu) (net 9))
 (segment (start 118.445 70.95) (end 122.385 70.95) (width 0.25) (layer F.Cu) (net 8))
 (segment (start 137.16 71.755) (end 137.16 70.485) (width 0.25) (layer F.Cu) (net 8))
 (segment (start 136.525 72.39) (end 137.16 71.755) (width 0.25) (layer F.Cu) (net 8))
 (segment (start 123.825 72.39) (end 136.525 72.39) (width 0.25) (layer F.Cu) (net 8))
 (segment (start 122.385 70.95) (end 123.825 72.39) (width 0.25) (layer F.Cu) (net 8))
 (segment (start 137.795 64.77) (end 137.795 69.85) (width 0.25) (layer F.Cu) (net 8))
 (segment (start 137.795 69.85) (end 137.16 70.485) (width 0.25) (layer F.Cu) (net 8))
 (segment (start 127.635 64.77) (end 127.635 68.58) (width 0.25) (layer F.Cu) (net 10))
 (segment (start 127.635 68.58) (end 125.73 70.485) (width 0.25) (layer F.Cu) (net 10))
 (segment (start 121.285 69.565) (end 123.54 69.565) (width 0.25) (layer F.Cu) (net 5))
 (segment (start 128.905 71.755) (end 124.46 71.755) (width 0.25) (layer F.Cu) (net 5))
 (segment (start 128.905 71.755) (end 129.54 71.12) (width 0.25) (layer F.Cu) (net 5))
 (segment (start 123.825 71.12) (end 124.46 71.755) (width 0.25) (layer F.Cu) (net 5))
 (segment (start 123.825 69.85) (end 123.825 71.12) (width 0.25) (layer F.Cu) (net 5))
 (segment (start 123.54 69.565) (end 123.825 69.85) (width 0.25) (layer F.Cu) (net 5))
 (segment (start 129.54 70.485) (end 129.54 71.12) (width 0.25) (layer F.Cu) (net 5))
 (segment (start 130.175 64.77) (end 130.175 69.85) (width 0.25) (layer F.Cu) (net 5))
 (segment (start 130.175 69.85) (end 129.54 70.485) (width 0.25) (layer F.Cu) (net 5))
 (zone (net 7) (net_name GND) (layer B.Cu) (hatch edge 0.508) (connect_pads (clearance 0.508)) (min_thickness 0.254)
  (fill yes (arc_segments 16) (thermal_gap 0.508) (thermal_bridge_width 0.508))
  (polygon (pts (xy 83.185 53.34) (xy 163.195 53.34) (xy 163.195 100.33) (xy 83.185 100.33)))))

